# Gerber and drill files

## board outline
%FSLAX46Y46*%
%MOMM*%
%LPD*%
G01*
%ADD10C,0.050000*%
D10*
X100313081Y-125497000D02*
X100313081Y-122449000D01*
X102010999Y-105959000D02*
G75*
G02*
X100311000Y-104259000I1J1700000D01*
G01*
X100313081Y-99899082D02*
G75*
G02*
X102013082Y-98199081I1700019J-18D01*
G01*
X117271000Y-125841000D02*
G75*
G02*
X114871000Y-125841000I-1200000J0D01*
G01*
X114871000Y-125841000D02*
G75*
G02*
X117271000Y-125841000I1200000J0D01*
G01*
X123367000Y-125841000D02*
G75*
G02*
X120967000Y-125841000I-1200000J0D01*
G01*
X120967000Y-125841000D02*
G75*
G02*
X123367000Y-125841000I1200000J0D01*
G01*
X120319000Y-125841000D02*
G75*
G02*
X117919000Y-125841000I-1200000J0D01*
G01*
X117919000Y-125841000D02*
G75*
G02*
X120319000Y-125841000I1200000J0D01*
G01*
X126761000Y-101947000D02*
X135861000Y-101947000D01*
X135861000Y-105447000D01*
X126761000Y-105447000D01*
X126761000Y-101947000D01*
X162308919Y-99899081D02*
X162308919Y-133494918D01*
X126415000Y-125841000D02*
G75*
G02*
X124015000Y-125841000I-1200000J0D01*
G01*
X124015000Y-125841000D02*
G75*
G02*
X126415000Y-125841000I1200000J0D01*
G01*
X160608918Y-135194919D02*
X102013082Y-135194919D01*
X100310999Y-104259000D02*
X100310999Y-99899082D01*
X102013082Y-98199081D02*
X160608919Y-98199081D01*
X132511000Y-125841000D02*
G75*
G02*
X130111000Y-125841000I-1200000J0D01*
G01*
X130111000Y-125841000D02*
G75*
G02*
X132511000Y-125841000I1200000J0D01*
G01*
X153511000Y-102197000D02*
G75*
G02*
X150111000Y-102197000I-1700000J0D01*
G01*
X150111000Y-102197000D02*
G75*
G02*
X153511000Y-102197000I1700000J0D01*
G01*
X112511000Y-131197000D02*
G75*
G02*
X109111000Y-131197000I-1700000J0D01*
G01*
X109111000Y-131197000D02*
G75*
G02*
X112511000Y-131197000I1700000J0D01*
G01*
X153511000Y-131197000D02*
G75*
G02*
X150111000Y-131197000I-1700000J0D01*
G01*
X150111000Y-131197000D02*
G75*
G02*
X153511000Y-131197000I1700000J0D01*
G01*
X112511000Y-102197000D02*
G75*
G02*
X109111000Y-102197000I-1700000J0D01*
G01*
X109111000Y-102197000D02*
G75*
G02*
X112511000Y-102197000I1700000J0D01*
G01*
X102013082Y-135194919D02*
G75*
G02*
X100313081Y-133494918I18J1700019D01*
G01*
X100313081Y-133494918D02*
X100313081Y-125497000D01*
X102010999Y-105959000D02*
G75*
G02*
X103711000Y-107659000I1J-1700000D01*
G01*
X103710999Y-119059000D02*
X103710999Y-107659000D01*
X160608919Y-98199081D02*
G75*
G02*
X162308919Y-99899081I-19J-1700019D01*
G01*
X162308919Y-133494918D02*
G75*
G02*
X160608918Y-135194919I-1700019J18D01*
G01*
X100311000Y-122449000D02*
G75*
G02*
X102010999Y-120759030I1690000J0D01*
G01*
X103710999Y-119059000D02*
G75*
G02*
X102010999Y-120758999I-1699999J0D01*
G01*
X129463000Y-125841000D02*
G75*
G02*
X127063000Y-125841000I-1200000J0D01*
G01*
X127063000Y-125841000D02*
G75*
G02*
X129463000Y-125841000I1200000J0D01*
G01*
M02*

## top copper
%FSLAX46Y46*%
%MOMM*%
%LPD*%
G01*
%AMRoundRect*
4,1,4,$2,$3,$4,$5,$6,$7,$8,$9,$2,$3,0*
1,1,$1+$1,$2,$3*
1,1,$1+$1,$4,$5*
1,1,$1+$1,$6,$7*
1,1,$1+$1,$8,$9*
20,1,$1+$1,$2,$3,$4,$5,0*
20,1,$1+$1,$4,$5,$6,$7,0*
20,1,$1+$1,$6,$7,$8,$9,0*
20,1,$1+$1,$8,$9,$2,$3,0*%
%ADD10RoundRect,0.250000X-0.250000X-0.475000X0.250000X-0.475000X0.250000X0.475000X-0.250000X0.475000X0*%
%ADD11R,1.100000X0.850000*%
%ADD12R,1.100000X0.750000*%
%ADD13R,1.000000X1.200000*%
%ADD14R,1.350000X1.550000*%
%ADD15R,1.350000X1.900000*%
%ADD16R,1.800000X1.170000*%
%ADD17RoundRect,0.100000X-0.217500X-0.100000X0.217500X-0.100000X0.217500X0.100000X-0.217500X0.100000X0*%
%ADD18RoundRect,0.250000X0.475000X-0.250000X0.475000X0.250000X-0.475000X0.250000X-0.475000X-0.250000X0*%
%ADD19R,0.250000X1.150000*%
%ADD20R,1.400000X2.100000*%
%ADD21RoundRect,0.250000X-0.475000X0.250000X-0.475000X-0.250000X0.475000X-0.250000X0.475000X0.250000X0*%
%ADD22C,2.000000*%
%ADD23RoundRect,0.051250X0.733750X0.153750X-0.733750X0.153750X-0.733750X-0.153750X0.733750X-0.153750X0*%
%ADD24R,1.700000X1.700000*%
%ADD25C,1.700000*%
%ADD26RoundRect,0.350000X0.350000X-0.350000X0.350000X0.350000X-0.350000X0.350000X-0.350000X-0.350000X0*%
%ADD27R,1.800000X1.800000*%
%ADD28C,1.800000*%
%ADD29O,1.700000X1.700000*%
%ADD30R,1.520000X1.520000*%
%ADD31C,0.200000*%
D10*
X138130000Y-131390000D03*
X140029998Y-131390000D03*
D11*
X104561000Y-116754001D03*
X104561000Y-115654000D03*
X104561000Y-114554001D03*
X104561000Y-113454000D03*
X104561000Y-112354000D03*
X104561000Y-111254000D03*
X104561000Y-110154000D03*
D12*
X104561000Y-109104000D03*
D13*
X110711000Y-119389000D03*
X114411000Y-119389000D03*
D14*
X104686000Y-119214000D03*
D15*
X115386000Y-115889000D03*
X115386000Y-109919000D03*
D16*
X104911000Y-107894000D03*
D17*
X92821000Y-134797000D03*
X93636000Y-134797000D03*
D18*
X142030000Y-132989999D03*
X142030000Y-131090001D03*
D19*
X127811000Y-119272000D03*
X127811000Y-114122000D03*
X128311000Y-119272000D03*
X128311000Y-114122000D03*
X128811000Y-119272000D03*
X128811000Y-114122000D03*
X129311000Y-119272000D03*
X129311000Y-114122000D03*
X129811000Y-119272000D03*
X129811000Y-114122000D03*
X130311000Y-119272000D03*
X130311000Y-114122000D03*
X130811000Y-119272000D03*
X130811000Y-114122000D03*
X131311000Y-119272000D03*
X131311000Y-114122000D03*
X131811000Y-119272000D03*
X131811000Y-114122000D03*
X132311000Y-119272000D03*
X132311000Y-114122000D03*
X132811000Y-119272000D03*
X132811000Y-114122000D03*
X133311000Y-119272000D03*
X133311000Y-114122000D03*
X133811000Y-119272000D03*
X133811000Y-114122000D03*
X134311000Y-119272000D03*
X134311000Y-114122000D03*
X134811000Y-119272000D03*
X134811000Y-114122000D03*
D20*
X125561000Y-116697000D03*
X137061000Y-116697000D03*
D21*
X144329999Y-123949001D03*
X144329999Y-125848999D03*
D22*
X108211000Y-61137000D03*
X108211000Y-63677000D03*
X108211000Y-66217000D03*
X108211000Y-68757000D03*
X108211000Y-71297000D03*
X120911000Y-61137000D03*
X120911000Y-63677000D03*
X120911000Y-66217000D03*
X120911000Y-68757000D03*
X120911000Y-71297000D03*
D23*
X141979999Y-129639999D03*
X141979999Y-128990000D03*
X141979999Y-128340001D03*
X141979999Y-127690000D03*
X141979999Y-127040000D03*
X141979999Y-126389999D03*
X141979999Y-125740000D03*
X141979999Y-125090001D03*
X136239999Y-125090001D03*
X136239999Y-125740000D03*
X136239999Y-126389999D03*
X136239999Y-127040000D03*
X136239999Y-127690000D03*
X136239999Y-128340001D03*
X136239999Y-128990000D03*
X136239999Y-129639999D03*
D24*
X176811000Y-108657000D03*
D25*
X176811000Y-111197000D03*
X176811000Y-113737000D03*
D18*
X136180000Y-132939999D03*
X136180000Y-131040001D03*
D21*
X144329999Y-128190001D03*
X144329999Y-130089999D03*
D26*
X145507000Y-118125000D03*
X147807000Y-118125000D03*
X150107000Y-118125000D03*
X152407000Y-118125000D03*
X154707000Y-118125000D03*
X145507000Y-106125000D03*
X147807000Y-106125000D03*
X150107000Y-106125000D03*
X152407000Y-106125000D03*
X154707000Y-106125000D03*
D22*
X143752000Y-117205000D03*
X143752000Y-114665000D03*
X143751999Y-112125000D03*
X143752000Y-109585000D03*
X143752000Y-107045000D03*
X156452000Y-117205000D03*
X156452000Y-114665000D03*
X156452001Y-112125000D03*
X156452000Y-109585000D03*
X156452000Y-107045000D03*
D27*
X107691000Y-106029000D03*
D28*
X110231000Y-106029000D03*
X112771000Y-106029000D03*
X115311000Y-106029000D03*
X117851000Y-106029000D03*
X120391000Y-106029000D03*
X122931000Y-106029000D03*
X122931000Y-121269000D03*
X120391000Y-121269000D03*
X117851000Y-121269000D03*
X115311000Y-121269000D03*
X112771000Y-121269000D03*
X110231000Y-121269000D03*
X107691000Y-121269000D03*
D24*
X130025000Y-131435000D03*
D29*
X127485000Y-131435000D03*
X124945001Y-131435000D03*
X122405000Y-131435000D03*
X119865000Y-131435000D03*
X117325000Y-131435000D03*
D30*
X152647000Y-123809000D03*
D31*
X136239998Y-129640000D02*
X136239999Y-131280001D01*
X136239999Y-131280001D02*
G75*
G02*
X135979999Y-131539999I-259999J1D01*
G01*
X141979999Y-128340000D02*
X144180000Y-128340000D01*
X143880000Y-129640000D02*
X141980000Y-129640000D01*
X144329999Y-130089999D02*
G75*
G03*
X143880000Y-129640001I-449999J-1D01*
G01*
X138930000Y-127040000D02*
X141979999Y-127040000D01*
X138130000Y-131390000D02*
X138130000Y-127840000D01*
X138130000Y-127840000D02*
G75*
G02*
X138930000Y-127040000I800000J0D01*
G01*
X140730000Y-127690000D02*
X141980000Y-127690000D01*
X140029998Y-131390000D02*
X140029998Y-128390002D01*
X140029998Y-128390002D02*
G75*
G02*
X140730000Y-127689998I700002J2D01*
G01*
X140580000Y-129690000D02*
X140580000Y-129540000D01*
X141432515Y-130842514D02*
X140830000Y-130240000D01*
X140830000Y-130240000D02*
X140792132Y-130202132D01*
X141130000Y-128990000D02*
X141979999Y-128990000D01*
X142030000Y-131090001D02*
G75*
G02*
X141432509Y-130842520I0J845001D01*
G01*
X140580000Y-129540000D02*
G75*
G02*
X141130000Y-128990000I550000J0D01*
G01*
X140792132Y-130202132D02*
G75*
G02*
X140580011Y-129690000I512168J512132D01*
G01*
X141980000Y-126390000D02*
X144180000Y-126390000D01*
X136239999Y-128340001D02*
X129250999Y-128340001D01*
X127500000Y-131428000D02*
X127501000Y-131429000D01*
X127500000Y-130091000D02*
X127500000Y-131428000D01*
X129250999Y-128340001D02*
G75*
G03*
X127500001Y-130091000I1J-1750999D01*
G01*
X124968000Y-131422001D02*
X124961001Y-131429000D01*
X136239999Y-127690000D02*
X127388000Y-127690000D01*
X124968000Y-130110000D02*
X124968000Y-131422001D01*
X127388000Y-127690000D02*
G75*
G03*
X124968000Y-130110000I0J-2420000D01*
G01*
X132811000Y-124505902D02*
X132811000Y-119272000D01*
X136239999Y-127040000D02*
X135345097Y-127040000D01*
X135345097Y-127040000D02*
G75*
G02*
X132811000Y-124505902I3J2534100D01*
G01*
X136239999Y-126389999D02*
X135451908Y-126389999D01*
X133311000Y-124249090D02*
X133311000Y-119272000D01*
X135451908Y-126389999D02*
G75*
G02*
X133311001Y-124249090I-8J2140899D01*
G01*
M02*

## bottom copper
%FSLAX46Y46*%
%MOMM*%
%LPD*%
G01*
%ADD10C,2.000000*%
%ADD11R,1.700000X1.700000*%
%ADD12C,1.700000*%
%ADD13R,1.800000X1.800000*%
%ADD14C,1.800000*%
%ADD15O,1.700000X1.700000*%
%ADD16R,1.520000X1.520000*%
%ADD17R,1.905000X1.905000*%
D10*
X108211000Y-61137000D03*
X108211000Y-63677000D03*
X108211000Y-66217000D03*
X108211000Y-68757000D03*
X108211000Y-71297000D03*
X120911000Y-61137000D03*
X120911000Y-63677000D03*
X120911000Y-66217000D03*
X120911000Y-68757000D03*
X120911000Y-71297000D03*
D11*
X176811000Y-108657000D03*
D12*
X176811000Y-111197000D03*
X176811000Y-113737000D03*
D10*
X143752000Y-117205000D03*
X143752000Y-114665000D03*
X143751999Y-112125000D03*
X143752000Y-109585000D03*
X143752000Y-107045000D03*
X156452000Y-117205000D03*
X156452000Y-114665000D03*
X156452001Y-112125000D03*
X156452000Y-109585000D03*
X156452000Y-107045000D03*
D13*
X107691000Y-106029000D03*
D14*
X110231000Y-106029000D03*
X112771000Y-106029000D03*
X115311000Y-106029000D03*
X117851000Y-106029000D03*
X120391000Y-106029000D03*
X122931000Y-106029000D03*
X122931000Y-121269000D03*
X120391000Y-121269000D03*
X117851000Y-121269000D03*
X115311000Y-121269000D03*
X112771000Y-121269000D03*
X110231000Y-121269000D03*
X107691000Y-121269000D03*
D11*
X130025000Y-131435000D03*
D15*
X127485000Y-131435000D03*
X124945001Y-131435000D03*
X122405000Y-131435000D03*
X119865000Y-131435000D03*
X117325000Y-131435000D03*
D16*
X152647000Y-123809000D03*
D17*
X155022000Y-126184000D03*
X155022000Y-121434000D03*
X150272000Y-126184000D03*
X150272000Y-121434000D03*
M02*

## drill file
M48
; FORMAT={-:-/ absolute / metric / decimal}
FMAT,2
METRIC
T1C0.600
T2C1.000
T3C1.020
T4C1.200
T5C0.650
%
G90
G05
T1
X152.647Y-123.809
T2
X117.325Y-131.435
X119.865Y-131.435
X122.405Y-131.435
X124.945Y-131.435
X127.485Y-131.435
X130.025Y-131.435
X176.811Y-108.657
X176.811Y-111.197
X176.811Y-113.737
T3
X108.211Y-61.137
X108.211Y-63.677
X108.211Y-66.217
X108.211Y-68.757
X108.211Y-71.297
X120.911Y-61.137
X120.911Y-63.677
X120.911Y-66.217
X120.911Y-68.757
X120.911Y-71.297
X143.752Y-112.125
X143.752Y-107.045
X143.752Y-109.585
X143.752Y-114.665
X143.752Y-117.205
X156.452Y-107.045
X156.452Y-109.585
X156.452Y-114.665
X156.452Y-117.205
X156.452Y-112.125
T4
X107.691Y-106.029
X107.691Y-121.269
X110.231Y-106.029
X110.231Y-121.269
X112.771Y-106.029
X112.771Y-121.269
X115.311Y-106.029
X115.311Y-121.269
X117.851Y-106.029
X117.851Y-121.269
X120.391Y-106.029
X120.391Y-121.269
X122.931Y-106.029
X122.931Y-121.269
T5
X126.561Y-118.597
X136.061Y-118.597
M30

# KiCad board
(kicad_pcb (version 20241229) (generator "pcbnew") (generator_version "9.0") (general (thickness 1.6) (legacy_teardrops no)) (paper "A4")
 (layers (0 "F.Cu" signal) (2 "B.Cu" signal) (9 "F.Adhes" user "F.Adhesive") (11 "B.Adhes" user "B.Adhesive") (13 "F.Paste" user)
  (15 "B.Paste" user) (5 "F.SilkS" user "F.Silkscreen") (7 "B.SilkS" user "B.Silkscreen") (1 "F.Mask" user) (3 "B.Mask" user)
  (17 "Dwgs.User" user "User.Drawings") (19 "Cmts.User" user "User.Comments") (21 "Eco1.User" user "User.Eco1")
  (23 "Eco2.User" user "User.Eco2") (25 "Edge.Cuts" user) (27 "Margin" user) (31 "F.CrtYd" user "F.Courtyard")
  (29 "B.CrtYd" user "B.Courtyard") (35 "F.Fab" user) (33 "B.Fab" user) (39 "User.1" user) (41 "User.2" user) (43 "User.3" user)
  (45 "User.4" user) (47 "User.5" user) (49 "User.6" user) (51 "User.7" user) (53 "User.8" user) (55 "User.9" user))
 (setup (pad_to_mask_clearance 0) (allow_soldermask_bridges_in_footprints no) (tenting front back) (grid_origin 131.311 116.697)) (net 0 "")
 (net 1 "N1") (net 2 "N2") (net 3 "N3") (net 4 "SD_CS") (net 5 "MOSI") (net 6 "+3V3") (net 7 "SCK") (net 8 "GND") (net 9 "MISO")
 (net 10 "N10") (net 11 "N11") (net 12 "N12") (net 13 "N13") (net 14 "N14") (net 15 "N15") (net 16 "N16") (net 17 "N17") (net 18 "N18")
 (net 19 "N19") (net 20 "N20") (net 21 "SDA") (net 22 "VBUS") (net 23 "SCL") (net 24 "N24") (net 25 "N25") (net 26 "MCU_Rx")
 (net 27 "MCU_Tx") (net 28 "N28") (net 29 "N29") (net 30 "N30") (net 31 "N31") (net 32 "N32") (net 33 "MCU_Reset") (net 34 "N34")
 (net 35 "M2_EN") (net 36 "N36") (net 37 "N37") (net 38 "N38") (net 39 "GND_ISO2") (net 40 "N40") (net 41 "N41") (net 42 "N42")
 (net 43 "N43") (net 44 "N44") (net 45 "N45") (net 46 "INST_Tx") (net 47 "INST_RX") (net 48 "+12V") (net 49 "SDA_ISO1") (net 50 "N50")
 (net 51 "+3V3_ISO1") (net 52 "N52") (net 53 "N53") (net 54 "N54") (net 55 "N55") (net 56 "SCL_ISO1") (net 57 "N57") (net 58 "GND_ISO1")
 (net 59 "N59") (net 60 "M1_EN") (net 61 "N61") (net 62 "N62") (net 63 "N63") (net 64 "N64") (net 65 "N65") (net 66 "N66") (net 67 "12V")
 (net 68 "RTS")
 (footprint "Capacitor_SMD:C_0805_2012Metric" (layer "F.Cu") (at 139.079999 131.39)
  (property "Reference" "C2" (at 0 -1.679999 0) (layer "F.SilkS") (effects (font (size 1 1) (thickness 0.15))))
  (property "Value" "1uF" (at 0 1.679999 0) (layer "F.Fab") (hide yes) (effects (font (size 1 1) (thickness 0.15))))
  (pad "1" smd roundrect (at -0.949999 0) (size 1 1.45) (layers "F.Cu" "F.Mask" "F.Paste") (roundrect_rratio 0.25) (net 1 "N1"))
  (pad "2" smd roundrect (at 0.949999 0) (size 1 1.45) (layers "F.Cu" "F.Mask" "F.Paste") (roundrect_rratio 0.25) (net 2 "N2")))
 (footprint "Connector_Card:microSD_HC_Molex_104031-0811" (layer "F.Cu") (at 110.011 113.649 90)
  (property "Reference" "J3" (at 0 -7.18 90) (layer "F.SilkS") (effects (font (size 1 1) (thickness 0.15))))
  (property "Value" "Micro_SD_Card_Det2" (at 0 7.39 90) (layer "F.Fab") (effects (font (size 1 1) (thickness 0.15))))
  (pad "1" smd rect (at -3.105001 -5.45 90) (size 0.85 1.1) (layers "F.Cu" "F.Mask" "F.Paste") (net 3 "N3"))
  (pad "2" smd rect (at -2.005 -5.45 90) (size 0.85 1.1) (layers "F.Cu" "F.Mask" "F.Paste") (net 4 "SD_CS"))
  (pad "3" smd rect (at -0.905001 -5.45 90) (size 0.85 1.1) (layers "F.Cu" "F.Mask" "F.Paste") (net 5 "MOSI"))
  (pad "4" smd rect (at 0.195 -5.45 90) (size 0.85 1.1) (layers "F.Cu" "F.Mask" "F.Paste") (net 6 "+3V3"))
  (pad "5" smd rect (at 1.295 -5.45 90) (size 0.85 1.1) (layers "F.Cu" "F.Mask" "F.Paste") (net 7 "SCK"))
  (pad "6" smd rect (at 2.395 -5.45 90) (size 0.85 1.1) (layers "F.Cu" "F.Mask" "F.Paste") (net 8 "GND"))
  (pad "7" smd rect (at 3.495 -5.45 90) (size 0.85 1.1) (layers "F.Cu" "F.Mask" "F.Paste") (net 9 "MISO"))
  (pad "8" smd rect (at 4.545 -5.45 90) (size 0.75 1.1) (layers "F.Cu" "F.Mask" "F.Paste") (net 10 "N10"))
  (pad "9" smd rect (at -5.74 0.7 90) (size 1.2 1) (layers "F.Cu" "F.Mask" "F.Paste") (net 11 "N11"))
  (pad "10" smd rect (at -5.74 4.4 90) (size 1.2 1) (layers "F.Cu" "F.Mask" "F.Paste") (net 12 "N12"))
  (pad "11" smd rect (at -5.565 -5.325 90) (size 1.55 1.35) (layers "F.Cu" "F.Mask" "F.Paste") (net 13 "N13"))
  (pad "11" smd rect (at -2.24 5.375 90) (size 1.9 1.35) (layers "F.Cu" "F.Mask" "F.Paste") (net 13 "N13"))
  (pad "11" smd rect (at 3.73 5.375 90) (size 1.9 1.35) (layers "F.Cu" "F.Mask" "F.Paste") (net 13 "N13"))
  (pad "11" smd rect (at 5.755 -5.1 90) (size 1.17 1.8) (layers "F.Cu" "F.Mask" "F.Paste") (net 13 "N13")))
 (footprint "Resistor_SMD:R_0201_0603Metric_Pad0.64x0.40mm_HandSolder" (layer "F.Cu") (at 93.2285 134.797)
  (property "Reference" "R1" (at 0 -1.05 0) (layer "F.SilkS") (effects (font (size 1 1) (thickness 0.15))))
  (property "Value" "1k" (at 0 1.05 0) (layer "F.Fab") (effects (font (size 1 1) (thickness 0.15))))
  (pad "" smd roundrect (at -0.4325 0) (size 0.458 0.36) (layers "F.Paste") (roundrect_rratio 0.25))
  (pad "" smd roundrect (at 0.4325 0) (size 0.458 0.36) (layers "F.Paste") (roundrect_rratio 0.25))
  (pad "1" smd roundrect (at -0.4075 0) (size 0.635 0.4) (layers "F.Cu" "F.Mask") (roundrect_rratio 0.25) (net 6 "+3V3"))
  (pad "2" smd roundrect (at 0.4075 0) (size 0.635 0.4) (layers "F.Cu" "F.Mask") (roundrect_rratio 0.25) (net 3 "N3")))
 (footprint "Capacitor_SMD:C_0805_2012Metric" (layer "F.Cu") (at 142.03 132.04 90)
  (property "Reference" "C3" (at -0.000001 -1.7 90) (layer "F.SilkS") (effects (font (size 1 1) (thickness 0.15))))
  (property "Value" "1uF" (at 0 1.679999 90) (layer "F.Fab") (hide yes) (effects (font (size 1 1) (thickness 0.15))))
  (pad "1" smd roundrect (at -0.949999 0 90) (size 1 1.45) (layers "F.Cu" "F.Mask" "F.Paste") (roundrect_rratio 0.25) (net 8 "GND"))
  (pad "2" smd roundrect (at 0.949999 0 90) (size 1 1.45) (layers "F.Cu" "F.Mask" "F.Paste") (roundrect_rratio 0.25) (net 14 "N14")))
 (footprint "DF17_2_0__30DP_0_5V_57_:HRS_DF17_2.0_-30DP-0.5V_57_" (layer "F.Cu") (at 131.311 116.697)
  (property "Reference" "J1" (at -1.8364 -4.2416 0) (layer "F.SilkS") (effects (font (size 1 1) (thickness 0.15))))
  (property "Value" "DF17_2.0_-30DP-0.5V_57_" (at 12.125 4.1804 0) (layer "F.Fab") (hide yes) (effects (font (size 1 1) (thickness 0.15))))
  (pad "" np_thru_hole circle (at -4.75 1.9) (size 0.65 0.65) (drill 0.65) (layers "*.Cu" "*.Mask"))
  (pad "" np_thru_hole circle (at 4.75 1.9) (size 0.65 0.65) (drill 0.65) (layers "*.Cu" "*.Mask"))
  (pad "1" smd rect (at -3.5 2.575) (size 0.25 1.15) (layers "F.Cu" "F.Mask" "F.Paste") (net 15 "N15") (solder_mask_margin 0.102))
  (pad "2" smd rect (at -3.5 -2.575) (size 0.25 1.15) (layers "F.Cu" "F.Mask" "F.Paste") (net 6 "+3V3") (solder_mask_margin 0.102))
  (pad "3" smd rect (at -3 2.575) (size 0.25 1.15) (layers "F.Cu" "F.Mask" "F.Paste") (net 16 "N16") (solder_mask_margin 0.102))
  (pad "4" smd rect (at -3 -2.575) (size 0.25 1.15) (layers "F.Cu" "F.Mask" "F.Paste") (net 6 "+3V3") (solder_mask_margin 0.102))
  (pad "5" smd rect (at -2.5 2.575) (size 0.25 1.15) (layers "F.Cu" "F.Mask" "F.Paste") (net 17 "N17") (solder_mask_margin 0.102))
  (pad "6" smd rect (at -2.5 -2.575) (size 0.25 1.15) (layers "F.Cu" "F.Mask" "F.Paste") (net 6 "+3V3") (solder_mask_margin 0.102))
  (pad "7" smd rect (at -2 2.575) (size 0.25 1.15) (layers "F.Cu" "F.Mask" "F.Paste") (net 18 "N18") (solder_mask_margin 0.102))
  (pad "8" smd rect (at -2 -2.575) (size 0.25 1.15) (layers "F.Cu" "F.Mask" "F.Paste") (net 8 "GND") (solder_mask_margin 0.102))
  (pad "9" smd rect (at -1.5 2.575) (size 0.25 1.15) (layers "F.Cu" "F.Mask" "F.Paste") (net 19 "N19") (solder_mask_margin 0.102))
  (pad "10" smd rect (at -1.5 -2.575) (size 0.25 1.15) (layers "F.Cu" "F.Mask" "F.Paste") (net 8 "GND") (solder_mask_margin 0.102))
  (pad "11" smd rect (at -1 2.575) (size 0.25 1.15) (layers "F.Cu" "F.Mask" "F.Paste") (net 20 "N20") (solder_mask_margin 0.102))
  (pad "12" smd rect (at -1 -2.575) (size 0.25 1.15) (layers "F.Cu" "F.Mask" "F.Paste") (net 8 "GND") (solder_mask_margin 0.102))
  (pad "13" smd rect (at -0.5 2.575) (size 0.25 1.15) (layers "F.Cu" "F.Mask" "F.Paste") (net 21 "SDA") (solder_mask_margin 0.102))
  (pad "14" smd rect (at -0.5 -2.575) (size 0.25 1.15) (layers "F.Cu" "F.Mask" "F.Paste") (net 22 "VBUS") (solder_mask_margin 0.102))
  (pad "15" smd rect (at 0 2.575) (size 0.25 1.15) (layers "F.Cu" "F.Mask" "F.Paste") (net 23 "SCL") (solder_mask_margin 0.102))
  (pad "16" smd rect (at 0 -2.575) (size 0.25 1.15) (layers "F.Cu" "F.Mask" "F.Paste") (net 22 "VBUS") (solder_mask_margin 0.102))
  (pad "17" smd rect (at 0.5 2.575) (size 0.25 1.15) (layers "F.Cu" "F.Mask" "F.Paste") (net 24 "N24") (solder_mask_margin 0.102))
  (pad "18" smd rect (at 0.5 -2.575) (size 0.25 1.15) (layers "F.Cu" "F.Mask" "F.Paste") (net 22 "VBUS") (solder_mask_margin 0.102))
  (pad "19" smd rect (at 1 2.575) (size 0.25 1.15) (layers "F.Cu" "F.Mask" "F.Paste") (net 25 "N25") (solder_mask_margin 0.102))
  (pad "20" smd rect (at 1 -2.575) (size 0.25 1.15) (layers "F.Cu" "F.Mask" "F.Paste") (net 8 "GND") (solder_mask_margin 0.102))
  (pad "21" smd rect (at 1.5 2.575) (size 0.25 1.15) (layers "F.Cu" "F.Mask" "F.Paste") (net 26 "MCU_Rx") (solder_mask_margin 0.102))
  (pad "22" smd rect (at 1.5 -2.575) (size 0.25 1.15) (layers "F.Cu" "F.Mask" "F.Paste") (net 8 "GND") (solder_mask_margin 0.102))
  (pad "23" smd rect (at 2 2.575) (size 0.25 1.15) (layers "F.Cu" "F.Mask" "F.Paste") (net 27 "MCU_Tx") (solder_mask_margin 0.102))
  (pad "24" smd rect (at 2 -2.575) (size 0.25 1.15) (layers "F.Cu" "F.Mask" "F.Paste") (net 8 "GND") (solder_mask_margin 0.102))
  (pad "25" smd rect (at 2.5 2.575) (size 0.25 1.15) (layers "F.Cu" "F.Mask" "F.Paste") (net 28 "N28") (solder_mask_margin 0.102))
  (pad "26" smd rect (at 2.5 -2.575) (size 0.25 1.15) (layers "F.Cu" "F.Mask" "F.Paste") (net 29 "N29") (solder_mask_margin 0.102))
  (pad "27" smd rect (at 3 2.575) (size 0.25 1.15) (layers "F.Cu" "F.Mask" "F.Paste") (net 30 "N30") (solder_mask_margin 0.102))
  (pad "28" smd rect (at 3 -2.575) (size 0.25 1.15) (layers "F.Cu" "F.Mask" "F.Paste") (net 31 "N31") (solder_mask_margin 0.102))
  (pad "29" smd rect (at 3.5 2.575) (size 0.25 1.15) (layers "F.Cu" "F.Mask" "F.Paste") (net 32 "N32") (solder_mask_margin 0.102))
  (pad "30" smd rect (at 3.5 -2.575) (size 0.25 1.15) (layers "F.Cu" "F.Mask" "F.Paste") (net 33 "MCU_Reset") (solder_mask_margin 0.102))
  (pad "S1" smd rect (at -5.75 0) (size 1.4 2.1) (layers "F.Cu" "F.Mask" "F.Paste") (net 8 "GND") (solder_mask_margin 0.102))
  (pad "S2" smd rect (at 5.75 0) (size 1.4 2.1) (layers "F.Cu" "F.Mask" "F.Paste") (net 8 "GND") (solder_mask_margin 0.102))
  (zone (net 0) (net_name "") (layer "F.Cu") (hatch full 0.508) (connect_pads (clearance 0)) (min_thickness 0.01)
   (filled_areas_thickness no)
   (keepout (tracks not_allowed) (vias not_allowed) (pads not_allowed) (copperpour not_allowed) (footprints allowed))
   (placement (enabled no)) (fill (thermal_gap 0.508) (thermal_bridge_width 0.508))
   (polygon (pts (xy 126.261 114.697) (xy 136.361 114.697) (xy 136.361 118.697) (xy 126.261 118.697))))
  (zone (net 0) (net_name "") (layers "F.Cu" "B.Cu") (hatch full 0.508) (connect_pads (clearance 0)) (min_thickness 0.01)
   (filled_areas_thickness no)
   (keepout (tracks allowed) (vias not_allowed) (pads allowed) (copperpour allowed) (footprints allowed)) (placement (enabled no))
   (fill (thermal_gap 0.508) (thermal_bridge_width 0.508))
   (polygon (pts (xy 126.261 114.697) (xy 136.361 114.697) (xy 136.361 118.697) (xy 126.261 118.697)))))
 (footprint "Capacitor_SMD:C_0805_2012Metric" (layer "F.Cu") (at 144.329999 124.899 -90)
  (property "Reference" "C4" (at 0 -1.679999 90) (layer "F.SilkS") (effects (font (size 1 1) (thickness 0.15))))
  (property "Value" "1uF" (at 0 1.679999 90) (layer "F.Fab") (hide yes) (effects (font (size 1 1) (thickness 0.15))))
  (pad "1" smd roundrect (at -0.949999 0 270) (size 1 1.45) (layers "F.Cu" "F.Mask" "F.Paste") (roundrect_rratio 0.25) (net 8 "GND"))
  (pad "2" smd roundrect (at 0.949999 0 270) (size 1 1.45) (layers "F.Cu" "F.Mask" "F.Paste") (roundrect_rratio 0.25) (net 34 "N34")))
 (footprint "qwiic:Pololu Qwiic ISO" (layer "F.Cu") (at 114.566 66.217)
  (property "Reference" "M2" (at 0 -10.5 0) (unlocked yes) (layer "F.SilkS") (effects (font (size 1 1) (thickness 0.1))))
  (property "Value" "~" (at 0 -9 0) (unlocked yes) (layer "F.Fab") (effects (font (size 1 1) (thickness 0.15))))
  (pad "1" thru_hole circle (at -6.355 -5.08) (size 2 2) (drill 1.02) (layers "*.Cu" "*.Mask") (remove_unused_layers no) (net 23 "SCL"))
  (pad "2" thru_hole circle (at -6.355 -2.54) (size 2 2) (drill 1.02) (layers "*.Cu" "*.Mask") (remove_unused_layers no) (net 21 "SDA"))
  (pad "3" thru_hole circle (at -6.355 0) (size 2 2) (drill 1.02) (layers "*.Cu" "*.Mask") (remove_unused_layers no) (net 6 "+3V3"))
  (pad "4" thru_hole circle (at -6.355 2.54) (size 2 2) (drill 1.02) (layers "*.Cu" "*.Mask") (remove_unused_layers no) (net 8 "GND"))
  (pad "5" thru_hole circle (at -6.355 5.08) (size 2 2) (drill 1.02) (layers "*.Cu" "*.Mask") (remove_unused_layers no) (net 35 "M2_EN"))
  (pad "6" thru_hole circle (at 6.345 -5.08) (size 2 2) (drill 1.02) (layers "*.Cu" "*.Mask") (remove_unused_layers no) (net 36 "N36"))
  (pad "7" thru_hole circle (at 6.345 -2.54) (size 2 2) (drill 1.02) (layers "*.Cu" "*.Mask") (remove_unused_layers no) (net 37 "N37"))
  (pad "8" thru_hole circle (at 6.345 0) (size 2 2) (drill 1.02) (layers "*.Cu" "*.Mask") (remove_unused_layers no) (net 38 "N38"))
  (pad "9" thru_hole circle (at 6.345 2.54) (size 2 2) (drill 1.02) (layers "*.Cu" "*.Mask") (remove_unused_layers no) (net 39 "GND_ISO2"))
  (pad "10" thru_hole circle (at 6.345 5.08) (size 2 2) (drill 1.02) (layers "*.Cu" "*.Mask") (remove_unused_layers no) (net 39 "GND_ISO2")))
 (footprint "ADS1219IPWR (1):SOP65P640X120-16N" (layer "F.Cu") (at 139.109999 127.365 180)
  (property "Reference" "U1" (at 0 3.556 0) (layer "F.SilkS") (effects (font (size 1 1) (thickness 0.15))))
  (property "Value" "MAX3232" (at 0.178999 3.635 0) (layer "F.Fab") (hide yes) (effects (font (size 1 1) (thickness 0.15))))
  (pad "1" smd roundrect (at -2.87 -2.274999 180) (size 1.57 0.41) (layers "F.Cu" "F.Mask" "F.Paste") (roundrect_rratio 0.125)
   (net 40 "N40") (solder_mask_margin 0.102))
  (pad "2" smd roundrect (at -2.87 -1.625 180) (size 1.57 0.41) (layers "F.Cu" "F.Mask" "F.Paste") (roundrect_rratio 0.125) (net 14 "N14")
   (solder_mask_margin 0.102))
  (pad "3" smd roundrect (at -2.87 -0.975001 180) (size 1.57 0.41) (layers "F.Cu" "F.Mask" "F.Paste") (roundrect_rratio 0.125)
   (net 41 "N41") (solder_mask_margin 0.102))
  (pad "4" smd roundrect (at -2.87 -0.325 180) (size 1.57 0.41) (layers "F.Cu" "F.Mask" "F.Paste") (roundrect_rratio 0.125) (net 2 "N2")
   (solder_mask_margin 0.102))
  (pad "5" smd roundrect (at -2.87 0.325 180) (size 1.57 0.41) (layers "F.Cu" "F.Mask" "F.Paste") (roundrect_rratio 0.125) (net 1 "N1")
   (solder_mask_margin 0.102))
  (pad "6" smd roundrect (at -2.87 0.975001 180) (size 1.57 0.41) (layers "F.Cu" "F.Mask" "F.Paste") (roundrect_rratio 0.125) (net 34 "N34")
   (solder_mask_margin 0.102))
  (pad "7" smd roundrect (at -2.87 1.625 180) (size 1.57 0.41) (layers "F.Cu" "F.Mask" "F.Paste") (roundrect_rratio 0.125) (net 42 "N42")
   (solder_mask_margin 0.102))
  (pad "8" smd roundrect (at -2.87 2.274999 180) (size 1.57 0.41) (layers "F.Cu" "F.Mask" "F.Paste") (roundrect_rratio 0.125) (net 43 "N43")
   (solder_mask_margin 0.102))
  (pad "9" smd roundrect (at 2.87 2.274999 180) (size 1.57 0.41) (layers "F.Cu" "F.Mask" "F.Paste") (roundrect_rratio 0.125) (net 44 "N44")
   (solder_mask_margin 0.102))
  (pad "10" smd roundrect (at 2.87 1.625 180) (size 1.57 0.41) (layers "F.Cu" "F.Mask" "F.Paste") (roundrect_rratio 0.125) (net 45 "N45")
   (solder_mask_margin 0.102))
  (pad "11" smd roundrect (at 2.87 0.975001 180) (size 1.57 0.41) (layers "F.Cu" "F.Mask" "F.Paste") (roundrect_rratio 0.125)
   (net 27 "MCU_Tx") (solder_mask_margin 0.102))
  (pad "12" smd roundrect (at 2.87 0.325 180) (size 1.57 0.41) (layers "F.Cu" "F.Mask" "F.Paste") (roundrect_rratio 0.125) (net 26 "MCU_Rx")
   (solder_mask_margin 0.102))
  (pad "13" smd roundrect (at 2.87 -0.325 180) (size 1.57 0.41) (layers "F.Cu" "F.Mask" "F.Paste") (roundrect_rratio 0.125)
   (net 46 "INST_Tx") (solder_mask_margin 0.102))
  (pad "14" smd roundrect (at 2.87 -0.975001 180) (size 1.57 0.41) (layers "F.Cu" "F.Mask" "F.Paste") (roundrect_rratio 0.125)
   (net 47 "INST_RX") (solder_mask_margin 0.102))
  (pad "15" smd roundrect (at 2.87 -1.625 180) (size 1.57 0.41) (layers "F.Cu" "F.Mask" "F.Paste") (roundrect_rratio 0.125) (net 8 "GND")
   (solder_mask_margin 0.102))
  (pad "16" smd roundrect (at 2.87 -2.274999 180) (size 1.57 0.41) (layers "F.Cu" "F.Mask" "F.Paste") (roundrect_rratio 0.125)
   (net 6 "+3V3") (solder_mask_margin 0.102)))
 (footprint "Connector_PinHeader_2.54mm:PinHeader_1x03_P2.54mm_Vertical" (layer "F.Cu") (at 176.811 108.657)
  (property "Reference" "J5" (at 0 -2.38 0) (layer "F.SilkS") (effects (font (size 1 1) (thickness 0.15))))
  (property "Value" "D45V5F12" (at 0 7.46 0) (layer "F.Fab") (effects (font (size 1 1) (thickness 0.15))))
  (pad "1" thru_hole rect (at 0 0) (size 1.7 1.7) (drill 1) (layers "*.Cu" "*.Mask") (remove_unused_layers no) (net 22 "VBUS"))
  (pad "2" thru_hole circle (at 0 2.54) (size 1.7 1.7) (drill 1) (layers "*.Cu" "*.Mask") (remove_unused_layers no) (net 8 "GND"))
  (pad "3" thru_hole circle (at 0 5.08) (size 1.7 1.7) (drill 1) (layers "*.Cu" "*.Mask") (remove_unused_layers no) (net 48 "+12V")))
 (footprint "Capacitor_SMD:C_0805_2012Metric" (layer "F.Cu") (at 136.18 131.99 90)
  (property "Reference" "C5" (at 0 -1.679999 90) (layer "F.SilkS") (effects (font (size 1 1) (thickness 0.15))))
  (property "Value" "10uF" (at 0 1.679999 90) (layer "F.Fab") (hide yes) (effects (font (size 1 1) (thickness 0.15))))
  (pad "1" smd roundrect (at -0.949999 0 90) (size 1 1.45) (layers "F.Cu" "F.Mask" "F.Paste") (roundrect_rratio 0.25) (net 8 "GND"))
  (pad "2" smd roundrect (at 0.949999 0 90) (size 1 1.45) (layers "F.Cu" "F.Mask" "F.Paste") (roundrect_rratio 0.25) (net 6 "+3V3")))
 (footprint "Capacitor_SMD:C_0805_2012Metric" (layer "F.Cu") (at 144.329999 129.14 -90)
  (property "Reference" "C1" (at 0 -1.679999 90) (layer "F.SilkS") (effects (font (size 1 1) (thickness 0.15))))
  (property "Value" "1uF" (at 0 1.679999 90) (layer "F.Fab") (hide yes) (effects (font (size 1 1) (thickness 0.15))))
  (pad "1" smd roundrect (at -0.949999 0 270) (size 1 1.45) (layers "F.Cu" "F.Mask" "F.Paste") (roundrect_rratio 0.25) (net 41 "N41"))
  (pad "2" smd roundrect (at 0.949999 0 270) (size 1 1.45) (layers "F.Cu" "F.Mask" "F.Paste") (roundrect_rratio 0.25) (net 40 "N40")))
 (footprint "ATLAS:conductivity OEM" (layer "F.Cu") (at 150.107 112.125 90)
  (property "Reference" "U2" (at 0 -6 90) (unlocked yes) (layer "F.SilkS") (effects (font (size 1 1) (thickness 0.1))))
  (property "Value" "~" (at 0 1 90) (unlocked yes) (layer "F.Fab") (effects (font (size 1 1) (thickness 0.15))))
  (pad "1" smd roundrect (at -6 -4.6 90) (size 1.4 1.4) (layers "F.Cu" "F.Mask" "F.Paste") (roundrect_rratio 0.25) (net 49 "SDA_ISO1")
   (thermal_bridge_angle 45))
  (pad "2" smd roundrect (at -6 -2.3 90) (size 1.4 1.4) (layers "F.Cu" "F.Mask" "F.Paste") (roundrect_rratio 0.25) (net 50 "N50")
   (thermal_bridge_angle 45))
  (pad "3" smd roundrect (at -6 0 90) (size 1.4 1.4) (layers "F.Cu" "F.Mask" "F.Paste") (roundrect_rratio 0.25) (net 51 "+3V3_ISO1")
   (thermal_bridge_angle 45))
  (pad "4" smd roundrect (at -6 2.3 90) (size 1.4 1.4) (layers "F.Cu" "F.Mask" "F.Paste") (roundrect_rratio 0.25) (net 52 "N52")
   (thermal_bridge_angle 45))
  (pad "5" smd roundrect (at -6 4.6 90) (size 1.4 1.4) (layers "F.Cu" "F.Mask" "F.Paste") (roundrect_rratio 0.25) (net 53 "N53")
   (thermal_bridge_angle 45))
  (pad "6" smd roundrect (at 6 -4.6 90) (size 1.4 1.4) (layers "F.Cu" "F.Mask" "F.Paste") (roundrect_rratio 0.25) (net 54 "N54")
   (thermal_bridge_angle 45))
  (pad "7" smd roundrect (at 6 -2.3 90) (size 1.4 1.4) (layers "F.Cu" "F.Mask" "F.Paste") (roundrect_rratio 0.25) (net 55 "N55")
   (thermal_bridge_angle 45))
  (pad "8" smd roundrect (at 6 0 90) (size 1.4 1.4) (layers "F.Cu" "F.Mask" "F.Paste") (roundrect_rratio 0.25) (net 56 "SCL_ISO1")
   (thermal_bridge_angle 45))
  (pad "9" smd roundrect (at 6 2.3 90) (size 1.4 1.4) (layers "F.Cu" "F.Mask" "F.Paste") (roundrect_rratio 0.25) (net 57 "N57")
   (thermal_bridge_angle 45))
  (pad "10" smd roundrect (at 6 4.6 90) (size 1.4 1.4) (layers "F.Cu" "F.Mask" "F.Paste") (roundrect_rratio 0.25) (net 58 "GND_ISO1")
   (thermal_bridge_angle 45)))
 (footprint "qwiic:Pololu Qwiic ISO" (layer "B.Cu") (at 150.107 112.125)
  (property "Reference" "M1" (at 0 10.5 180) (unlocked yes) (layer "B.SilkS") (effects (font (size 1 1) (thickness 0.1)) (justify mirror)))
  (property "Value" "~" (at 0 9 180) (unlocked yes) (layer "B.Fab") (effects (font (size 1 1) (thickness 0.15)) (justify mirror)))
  (pad "1" thru_hole circle (at -6.355 5.08) (size 2 2) (drill 1.02) (layers "*.Cu" "*.Mask") (remove_unused_layers no) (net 23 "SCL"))
  (pad "2" thru_hole circle (at -6.355 2.54) (size 2 2) (drill 1.02) (layers "*.Cu" "*.Mask") (remove_unused_layers no) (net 21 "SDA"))
  (pad "3" thru_hole circle (at -6.355001 0) (size 2 2) (drill 1.02) (layers "*.Cu" "*.Mask") (remove_unused_layers no) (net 6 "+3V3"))
  (pad "4" thru_hole circle (at -6.355 -2.54) (size 2 2) (drill 1.02) (layers "*.Cu" "*.Mask") (remove_unused_layers no) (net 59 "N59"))
  (pad "5" thru_hole circle (at -6.355 -5.08) (size 2 2) (drill 1.02) (layers "*.Cu" "*.Mask") (remove_unused_layers no) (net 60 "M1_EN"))
  (pad "6" thru_hole circle (at 6.345 5.08) (size 2 2) (drill 1.02) (layers "*.Cu" "*.Mask") (remove_unused_layers no) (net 56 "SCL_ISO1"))
  (pad "7" thru_hole circle (at 6.345 2.54) (size 2 2) (drill 1.02) (layers "*.Cu" "*.Mask") (remove_unused_layers no) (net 49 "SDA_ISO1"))
  (pad "8" thru_hole circle (at 6.345001 0) (size 2 2) (drill 1.02) (layers "*.Cu" "*.Mask") (remove_unused_layers no) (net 51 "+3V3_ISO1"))
  (pad "9" thru_hole circle (at 6.345 -2.54) (size 2 2) (drill 1.02) (layers "*.Cu" "*.Mask") (remove_unused_layers no) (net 58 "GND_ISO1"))
  (pad "10" thru_hole circle (at 6.345 -5.08) (size 2 2) (drill 1.02) (layers "*.Cu" "*.Mask") (remove_unused_layers no) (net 58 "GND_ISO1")))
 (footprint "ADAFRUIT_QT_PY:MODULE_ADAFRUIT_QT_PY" (layer "B.Cu") (at 115.311 113.649 -90)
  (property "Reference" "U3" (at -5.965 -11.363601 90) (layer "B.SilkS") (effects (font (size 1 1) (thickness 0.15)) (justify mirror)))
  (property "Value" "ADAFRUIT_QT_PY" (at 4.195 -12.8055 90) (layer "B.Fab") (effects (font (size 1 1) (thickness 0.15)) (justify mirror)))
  (pad "1" thru_hole rect (at -7.62 7.62 270) (size 1.8 1.8) (drill 1.2) (layers "*.Cu" "*.Mask") (remove_unused_layers no) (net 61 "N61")
   (solder_mask_margin 0.102))
  (pad "2" thru_hole circle (at -7.62 5.08 270) (size 1.8 1.8) (drill 1.2) (layers "*.Cu" "*.Mask") (remove_unused_layers no)
   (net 60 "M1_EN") (solder_mask_margin 0.102))
  (pad "3" thru_hole circle (at -7.62 2.54 270) (size 1.8 1.8) (drill 1.2) (layers "*.Cu" "*.Mask") (remove_unused_layers no)
   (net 35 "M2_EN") (solder_mask_margin 0.102))
  (pad "4" thru_hole circle (at -7.62 0 270) (size 1.8 1.8) (drill 1.2) (layers "*.Cu" "*.Mask") (remove_unused_layers no) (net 4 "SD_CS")
   (solder_mask_margin 0.102))
  (pad "5" thru_hole circle (at -7.62 -2.54 270) (size 1.8 1.8) (drill 1.2) (layers "*.Cu" "*.Mask") (remove_unused_layers no)
   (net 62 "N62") (solder_mask_margin 0.102))
  (pad "6" thru_hole circle (at -7.62 -5.08 270) (size 1.8 1.8) (drill 1.2) (layers "*.Cu" "*.Mask") (remove_unused_layers no)
   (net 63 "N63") (solder_mask_margin 0.102))
  (pad "7" thru_hole circle (at -7.62 -7.62 270) (size 1.8 1.8) (drill 1.2) (layers "*.Cu" "*.Mask") (remove_unused_layers no)
   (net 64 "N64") (solder_mask_margin 0.102))
  (pad "8" thru_hole circle (at 7.62 -7.62 270) (size 1.8 1.8) (drill 1.2) (layers "*.Cu" "*.Mask") (remove_unused_layers no) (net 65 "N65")
   (solder_mask_margin 0.102))
  (pad "9" thru_hole circle (at 7.62 -5.08 270) (size 1.8 1.8) (drill 1.2) (layers "*.Cu" "*.Mask") (remove_unused_layers no) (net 7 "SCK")
   (solder_mask_margin 0.102))
  (pad "10" thru_hole circle (at 7.62 -2.54 270) (size 1.8 1.8) (drill 1.2) (layers "*.Cu" "*.Mask") (remove_unused_layers no)
   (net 9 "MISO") (solder_mask_margin 0.102))
  (pad "11" thru_hole circle (at 7.62 0 270) (size 1.8 1.8) (drill 1.2) (layers "*.Cu" "*.Mask") (remove_unused_layers no) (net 5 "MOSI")
   (solder_mask_margin 0.102))
  (pad "12" thru_hole circle (at 7.62 2.54 270) (size 1.8 1.8) (drill 1.2) (layers "*.Cu" "*.Mask") (remove_unused_layers no) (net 6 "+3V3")
   (solder_mask_margin 0.102))
  (pad "13" thru_hole circle (at 7.62 5.08 270) (size 1.8 1.8) (drill 1.2) (layers "*.Cu" "*.Mask") (remove_unused_layers no) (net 8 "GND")
   (solder_mask_margin 0.102))
  (pad "14" thru_hole circle (at 7.62 7.62 270) (size 1.8 1.8) (drill 1.2) (layers "*.Cu" "*.Mask") (remove_unused_layers no) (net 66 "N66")
   (solder_mask_margin 0.102)))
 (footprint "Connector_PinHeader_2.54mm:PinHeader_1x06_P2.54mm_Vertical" (layer "B.Cu") (at 130.025 131.435 90)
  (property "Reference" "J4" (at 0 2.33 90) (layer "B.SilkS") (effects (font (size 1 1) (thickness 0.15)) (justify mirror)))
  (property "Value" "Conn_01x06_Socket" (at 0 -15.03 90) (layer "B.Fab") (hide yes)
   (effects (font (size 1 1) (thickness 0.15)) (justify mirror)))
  (pad "1" thru_hole rect (at 0 0 90) (size 1.7 1.7) (drill 1) (layers "*.Cu" "*.Mask") (remove_unused_layers no) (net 8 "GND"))
  (pad "2" thru_hole oval (at 0 -2.54 90) (size 1.7 1.7) (drill 1) (layers "*.Cu" "*.Mask") (remove_unused_layers no) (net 47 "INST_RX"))
  (pad "3" thru_hole oval (at 0 -5.079999 90) (size 1.7 1.7) (drill 1) (layers "*.Cu" "*.Mask") (remove_unused_layers no) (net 46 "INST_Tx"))
  (pad "4" thru_hole oval (at 0 -7.62 90) (size 1.7 1.7) (drill 1) (layers "*.Cu" "*.Mask") (remove_unused_layers no) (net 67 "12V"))
  (pad "5" thru_hole oval (at 0 -10.16 90) (size 1.7 1.7) (drill 1) (layers "*.Cu" "*.Mask") (remove_unused_layers no) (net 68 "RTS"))
  (pad "6" thru_hole oval (at 0 -12.7 90) (size 1.7 1.7) (drill 1) (layers "*.Cu" "*.Mask") (remove_unused_layers no) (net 8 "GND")))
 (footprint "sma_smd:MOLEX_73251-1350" (layer "B.Cu") (at 152.647 123.809 180)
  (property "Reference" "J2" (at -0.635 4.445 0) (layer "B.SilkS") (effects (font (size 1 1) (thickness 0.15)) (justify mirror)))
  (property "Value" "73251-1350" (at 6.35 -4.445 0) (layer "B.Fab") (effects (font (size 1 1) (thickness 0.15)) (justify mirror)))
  (pad "1" thru_hole rect (at 0 0 180) (size 1.52 1.52) (drill 0.6) (layers "*.Cu" "*.Mask") (remove_unused_layers no) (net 52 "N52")
   (solder_mask_margin 0.0762))
  (pad "S1" smd rect (at -2.375 -2.375 180) (size 1.905 1.905) (layers "B.Cu" "B.Mask" "B.Paste") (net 53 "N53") (solder_mask_margin 0.0762))
  (pad "S1" smd rect (at -2.375 2.375 180) (size 1.905 1.905) (layers "B.Cu" "B.Mask" "B.Paste") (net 53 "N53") (solder_mask_margin 0.0762))
  (pad "S1" smd rect (at 2.375 -2.375 180) (size 1.905 1.905) (layers "B.Cu" "B.Mask" "B.Paste") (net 53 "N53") (solder_mask_margin 0.0762))
  (pad "S1" smd rect (at 2.375 2.375 180) (size 1.905 1.905) (layers "B.Cu" "B.Mask" "B.Paste") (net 53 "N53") (solder_mask_margin 0.0762)))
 (gr_line (start 100.313081 125.497) (end 100.313081 122.449) (stroke (width 0.05) (type default)) (layer "Edge.Cuts"))
 (gr_arc (start 102.010999 105.959) (mid 100.808917 105.461082) (end 100.310999 104.259) (stroke (width 0.05) (type default))
  (layer "Edge.Cuts"))
 (gr_arc (start 100.313081 99.899082) (mid 100.811 98.697) (end 102.013082 98.199081) (stroke (width 0.05) (type default))
  (layer "Edge.Cuts"))
 (gr_circle (center 116.071 125.841) (end 117.271 125.841) (stroke (width 0.05) (type default)) (fill no) (layer "Edge.Cuts"))
 (gr_circle (center 122.167 125.841) (end 123.367 125.841) (stroke (width 0.05) (type default)) (fill no) (layer "Edge.Cuts"))
 (gr_circle (center 119.119 125.841) (end 120.319 125.841) (stroke (width 0.05) (type default)) (fill no) (layer "Edge.Cuts"))
 (gr_rect (start 126.761 101.947) (end 135.861 105.447) (stroke (width 0.05) (type default)) (fill no) (layer "Edge.Cuts"))
 (gr_line (start 162.308919 99.899081) (end 162.308919 133.494918) (stroke (width 0.05) (type default)) (layer "Edge.Cuts"))
 (gr_circle (center 125.215 125.841) (end 126.415 125.841) (stroke (width 0.05) (type default)) (fill no) (layer "Edge.Cuts"))
 (gr_line (start 160.608918 135.194919) (end 102.013082 135.194919) (stroke (width 0.05) (type default)) (layer "Edge.Cuts"))
 (gr_line (start 100.310999 104.259) (end 100.310999 99.899082) (stroke (width 0.05) (type default)) (layer "Edge.Cuts"))
 (gr_line (start 102.013082 98.199081) (end 160.608919 98.199081) (stroke (width 0.05) (type default)) (layer "Edge.Cuts"))
 (gr_circle (center 131.311 125.841) (end 132.511 125.841) (stroke (width 0.05) (type default)) (fill no) (layer "Edge.Cuts"))
 (gr_circle (center 151.811 102.197) (end 153.511 102.197) (stroke (width 0.05) (type default)) (fill no) (layer "Edge.Cuts"))
 (gr_circle (center 110.811 131.197) (end 112.511 131.197) (stroke (width 0.05) (type default)) (fill no) (layer "Edge.Cuts"))
 (gr_circle (center 151.811 131.197) (end 153.511 131.197) (stroke (width 0.05) (type default)) (fill no) (layer "Edge.Cuts"))
 (gr_circle (center 110.811 102.197) (end 112.511 102.197) (stroke (width 0.05) (type default)) (fill no) (layer "Edge.Cuts"))
 (gr_arc (start 102.013082 135.194919) (mid 100.811 134.697) (end 100.313081 133.494918) (stroke (width 0.05) (type default))
  (layer "Edge.Cuts"))
 (gr_line (start 100.313081 133.494918) (end 100.313081 125.497) (stroke (width 0.05) (type default)) (layer "Edge.Cuts"))
 (gr_arc (start 102.010999 105.959) (mid 103.21308 106.456919) (end 103.710999 107.659) (stroke (width 0.05) (type default))
  (layer "Edge.Cuts"))
 (gr_line (start 103.710999 119.059) (end 103.710999 107.659) (stroke (width 0.05) (type default)) (layer "Edge.Cuts"))
 (gr_arc (start 160.608919 98.199081) (mid 161.811 98.697) (end 162.308919 99.899081) (stroke (width 0.05) (type default))
  (layer "Edge.Cuts"))
 (gr_arc (start 162.308919 133.494918) (mid 161.811 134.697) (end 160.608918 135.194919) (stroke (width 0.05) (type default))
  (layer "Edge.Cuts"))
 (gr_arc (start 100.311 122.449) (mid 100.809528 121.250449) (end 102.010999 120.759) (stroke (width 0.05) (type default))
  (layer "Edge.Cuts"))
 (gr_arc (start 103.710999 119.059) (mid 103.213081 120.261082) (end 102.010999 120.759) (stroke (width 0.05) (type default))
  (layer "Edge.Cuts"))
 (gr_circle (center 128.263 125.841) (end 129.463 125.841) (stroke (width 0.05) (type default)) (fill no) (layer "Edge.Cuts"))
 (segment (start 136.239998 129.64) (end 136.239999 131.280001) (width 0.2) (layer "F.Cu") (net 6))
 (arc (start 136.239999 131.280001) (mid 136.163848 131.463848) (end 135.979999 131.54) (width 0.2) (layer "F.Cu") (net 6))
 (segment (start 141.979999 128.34) (end 144.18 128.34) (width 0.2) (layer "F.Cu") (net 41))
 (segment (start 143.88 129.64) (end 141.98 129.64) (width 0.2) (layer "F.Cu") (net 40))
 (arc (start 144.329999 130.089999) (mid 144.198197 129.771802) (end 143.88 129.64) (width 0.2) (layer "F.Cu") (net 40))
 (segment (start 138.93 127.04) (end 141.979999 127.04) (width 0.2) (layer "F.Cu") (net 1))
 (segment (start 138.13 131.39) (end 138.13 127.84) (width 0.2) (layer "F.Cu") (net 1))
 (arc (start 138.13 127.84) (mid 138.364315 127.274315) (end 138.93 127.04) (width 0.2) (layer "F.Cu") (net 1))
 (segment (start 140.73 127.69) (end 141.98 127.69) (width 0.2) (layer "F.Cu") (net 2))
 (segment (start 140.029998 131.39) (end 140.029998 128.390002) (width 0.2) (layer "F.Cu") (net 2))
 (arc (start 140.029998 128.390002) (mid 140.235024 127.895026) (end 140.73 127.69) (width 0.2) (layer "F.Cu") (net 2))
 (segment (start 140.58 129.69) (end 140.58 129.54) (width 0.2) (layer "F.Cu") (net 14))
 (segment (start 141.432515 130.842514) (end 140.83 130.24) (width 0.2) (layer "F.Cu") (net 14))
 (segment (start 140.83 130.24) (end 140.792132 130.202132) (width 0.2) (layer "F.Cu") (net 14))
 (segment (start 141.13 128.99) (end 141.979999 128.99) (width 0.2) (layer "F.Cu") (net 14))
 (arc (start 142.03 131.090001) (mid 141.706643 131.025681) (end 141.432515 130.842514) (width 0.2) (layer "F.Cu") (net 14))
 (arc (start 140.58 129.54) (mid 140.741091 129.151091) (end 141.13 128.99) (width 0.2) (layer "F.Cu") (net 14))
 (arc (start 140.792132 130.202132) (mid 140.635132 129.967164) (end 140.58 129.69) (width 0.2) (layer "F.Cu") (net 14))
 (segment (start 141.98 126.39) (end 144.18 126.39) (width 0.2) (layer "F.Cu") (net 34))
 (segment (start 136.239999 128.340001) (end 129.250999 128.340001) (width 0.2) (layer "F.Cu") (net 47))
 (segment (start 127.5 131.428) (end 127.501 131.429) (width 0.2) (layer "F.Cu") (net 47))
 (segment (start 127.5 130.091) (end 127.5 131.428) (width 0.2) (layer "F.Cu") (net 47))
 (arc (start 129.250999 128.340001) (mid 128.012856 128.852857) (end 127.5 130.091) (width 0.2) (layer "F.Cu") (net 47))
 (segment (start 124.968 131.422001) (end 124.961001 131.429) (width 0.2) (layer "F.Cu") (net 46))
 (segment (start 136.239999 127.69) (end 127.388 127.69) (width 0.2) (layer "F.Cu") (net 46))
 (segment (start 124.968 130.11) (end 124.968 131.422001) (width 0.2) (layer "F.Cu") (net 46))
 (arc (start 127.388 127.69) (mid 125.676802 128.398802) (end 124.968 130.11) (width 0.2) (layer "F.Cu") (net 46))
 (segment (start 132.811 124.505902) (end 132.811 119.272) (width 0.2) (layer "F.Cu") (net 26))
 (segment (start 136.239999 127.04) (end 135.345097 127.04) (width 0.2) (layer "F.Cu") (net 26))
 (arc (start 135.345097 127.04) (mid 133.55322 126.29778) (end 132.811 124.505902) (width 0.2) (layer "F.Cu") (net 26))
 (segment (start 136.239999 126.389999) (end 135.451908 126.389999) (width 0.2) (layer "F.Cu") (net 27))
 (segment (start 133.311 124.24909) (end 133.311 119.272) (width 0.2) (layer "F.Cu") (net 27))
 (arc (start 135.451908 126.389999) (mid 133.938057 125.762941) (end 133.311 124.24909) (width 0.2) (layer "F.Cu") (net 27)))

